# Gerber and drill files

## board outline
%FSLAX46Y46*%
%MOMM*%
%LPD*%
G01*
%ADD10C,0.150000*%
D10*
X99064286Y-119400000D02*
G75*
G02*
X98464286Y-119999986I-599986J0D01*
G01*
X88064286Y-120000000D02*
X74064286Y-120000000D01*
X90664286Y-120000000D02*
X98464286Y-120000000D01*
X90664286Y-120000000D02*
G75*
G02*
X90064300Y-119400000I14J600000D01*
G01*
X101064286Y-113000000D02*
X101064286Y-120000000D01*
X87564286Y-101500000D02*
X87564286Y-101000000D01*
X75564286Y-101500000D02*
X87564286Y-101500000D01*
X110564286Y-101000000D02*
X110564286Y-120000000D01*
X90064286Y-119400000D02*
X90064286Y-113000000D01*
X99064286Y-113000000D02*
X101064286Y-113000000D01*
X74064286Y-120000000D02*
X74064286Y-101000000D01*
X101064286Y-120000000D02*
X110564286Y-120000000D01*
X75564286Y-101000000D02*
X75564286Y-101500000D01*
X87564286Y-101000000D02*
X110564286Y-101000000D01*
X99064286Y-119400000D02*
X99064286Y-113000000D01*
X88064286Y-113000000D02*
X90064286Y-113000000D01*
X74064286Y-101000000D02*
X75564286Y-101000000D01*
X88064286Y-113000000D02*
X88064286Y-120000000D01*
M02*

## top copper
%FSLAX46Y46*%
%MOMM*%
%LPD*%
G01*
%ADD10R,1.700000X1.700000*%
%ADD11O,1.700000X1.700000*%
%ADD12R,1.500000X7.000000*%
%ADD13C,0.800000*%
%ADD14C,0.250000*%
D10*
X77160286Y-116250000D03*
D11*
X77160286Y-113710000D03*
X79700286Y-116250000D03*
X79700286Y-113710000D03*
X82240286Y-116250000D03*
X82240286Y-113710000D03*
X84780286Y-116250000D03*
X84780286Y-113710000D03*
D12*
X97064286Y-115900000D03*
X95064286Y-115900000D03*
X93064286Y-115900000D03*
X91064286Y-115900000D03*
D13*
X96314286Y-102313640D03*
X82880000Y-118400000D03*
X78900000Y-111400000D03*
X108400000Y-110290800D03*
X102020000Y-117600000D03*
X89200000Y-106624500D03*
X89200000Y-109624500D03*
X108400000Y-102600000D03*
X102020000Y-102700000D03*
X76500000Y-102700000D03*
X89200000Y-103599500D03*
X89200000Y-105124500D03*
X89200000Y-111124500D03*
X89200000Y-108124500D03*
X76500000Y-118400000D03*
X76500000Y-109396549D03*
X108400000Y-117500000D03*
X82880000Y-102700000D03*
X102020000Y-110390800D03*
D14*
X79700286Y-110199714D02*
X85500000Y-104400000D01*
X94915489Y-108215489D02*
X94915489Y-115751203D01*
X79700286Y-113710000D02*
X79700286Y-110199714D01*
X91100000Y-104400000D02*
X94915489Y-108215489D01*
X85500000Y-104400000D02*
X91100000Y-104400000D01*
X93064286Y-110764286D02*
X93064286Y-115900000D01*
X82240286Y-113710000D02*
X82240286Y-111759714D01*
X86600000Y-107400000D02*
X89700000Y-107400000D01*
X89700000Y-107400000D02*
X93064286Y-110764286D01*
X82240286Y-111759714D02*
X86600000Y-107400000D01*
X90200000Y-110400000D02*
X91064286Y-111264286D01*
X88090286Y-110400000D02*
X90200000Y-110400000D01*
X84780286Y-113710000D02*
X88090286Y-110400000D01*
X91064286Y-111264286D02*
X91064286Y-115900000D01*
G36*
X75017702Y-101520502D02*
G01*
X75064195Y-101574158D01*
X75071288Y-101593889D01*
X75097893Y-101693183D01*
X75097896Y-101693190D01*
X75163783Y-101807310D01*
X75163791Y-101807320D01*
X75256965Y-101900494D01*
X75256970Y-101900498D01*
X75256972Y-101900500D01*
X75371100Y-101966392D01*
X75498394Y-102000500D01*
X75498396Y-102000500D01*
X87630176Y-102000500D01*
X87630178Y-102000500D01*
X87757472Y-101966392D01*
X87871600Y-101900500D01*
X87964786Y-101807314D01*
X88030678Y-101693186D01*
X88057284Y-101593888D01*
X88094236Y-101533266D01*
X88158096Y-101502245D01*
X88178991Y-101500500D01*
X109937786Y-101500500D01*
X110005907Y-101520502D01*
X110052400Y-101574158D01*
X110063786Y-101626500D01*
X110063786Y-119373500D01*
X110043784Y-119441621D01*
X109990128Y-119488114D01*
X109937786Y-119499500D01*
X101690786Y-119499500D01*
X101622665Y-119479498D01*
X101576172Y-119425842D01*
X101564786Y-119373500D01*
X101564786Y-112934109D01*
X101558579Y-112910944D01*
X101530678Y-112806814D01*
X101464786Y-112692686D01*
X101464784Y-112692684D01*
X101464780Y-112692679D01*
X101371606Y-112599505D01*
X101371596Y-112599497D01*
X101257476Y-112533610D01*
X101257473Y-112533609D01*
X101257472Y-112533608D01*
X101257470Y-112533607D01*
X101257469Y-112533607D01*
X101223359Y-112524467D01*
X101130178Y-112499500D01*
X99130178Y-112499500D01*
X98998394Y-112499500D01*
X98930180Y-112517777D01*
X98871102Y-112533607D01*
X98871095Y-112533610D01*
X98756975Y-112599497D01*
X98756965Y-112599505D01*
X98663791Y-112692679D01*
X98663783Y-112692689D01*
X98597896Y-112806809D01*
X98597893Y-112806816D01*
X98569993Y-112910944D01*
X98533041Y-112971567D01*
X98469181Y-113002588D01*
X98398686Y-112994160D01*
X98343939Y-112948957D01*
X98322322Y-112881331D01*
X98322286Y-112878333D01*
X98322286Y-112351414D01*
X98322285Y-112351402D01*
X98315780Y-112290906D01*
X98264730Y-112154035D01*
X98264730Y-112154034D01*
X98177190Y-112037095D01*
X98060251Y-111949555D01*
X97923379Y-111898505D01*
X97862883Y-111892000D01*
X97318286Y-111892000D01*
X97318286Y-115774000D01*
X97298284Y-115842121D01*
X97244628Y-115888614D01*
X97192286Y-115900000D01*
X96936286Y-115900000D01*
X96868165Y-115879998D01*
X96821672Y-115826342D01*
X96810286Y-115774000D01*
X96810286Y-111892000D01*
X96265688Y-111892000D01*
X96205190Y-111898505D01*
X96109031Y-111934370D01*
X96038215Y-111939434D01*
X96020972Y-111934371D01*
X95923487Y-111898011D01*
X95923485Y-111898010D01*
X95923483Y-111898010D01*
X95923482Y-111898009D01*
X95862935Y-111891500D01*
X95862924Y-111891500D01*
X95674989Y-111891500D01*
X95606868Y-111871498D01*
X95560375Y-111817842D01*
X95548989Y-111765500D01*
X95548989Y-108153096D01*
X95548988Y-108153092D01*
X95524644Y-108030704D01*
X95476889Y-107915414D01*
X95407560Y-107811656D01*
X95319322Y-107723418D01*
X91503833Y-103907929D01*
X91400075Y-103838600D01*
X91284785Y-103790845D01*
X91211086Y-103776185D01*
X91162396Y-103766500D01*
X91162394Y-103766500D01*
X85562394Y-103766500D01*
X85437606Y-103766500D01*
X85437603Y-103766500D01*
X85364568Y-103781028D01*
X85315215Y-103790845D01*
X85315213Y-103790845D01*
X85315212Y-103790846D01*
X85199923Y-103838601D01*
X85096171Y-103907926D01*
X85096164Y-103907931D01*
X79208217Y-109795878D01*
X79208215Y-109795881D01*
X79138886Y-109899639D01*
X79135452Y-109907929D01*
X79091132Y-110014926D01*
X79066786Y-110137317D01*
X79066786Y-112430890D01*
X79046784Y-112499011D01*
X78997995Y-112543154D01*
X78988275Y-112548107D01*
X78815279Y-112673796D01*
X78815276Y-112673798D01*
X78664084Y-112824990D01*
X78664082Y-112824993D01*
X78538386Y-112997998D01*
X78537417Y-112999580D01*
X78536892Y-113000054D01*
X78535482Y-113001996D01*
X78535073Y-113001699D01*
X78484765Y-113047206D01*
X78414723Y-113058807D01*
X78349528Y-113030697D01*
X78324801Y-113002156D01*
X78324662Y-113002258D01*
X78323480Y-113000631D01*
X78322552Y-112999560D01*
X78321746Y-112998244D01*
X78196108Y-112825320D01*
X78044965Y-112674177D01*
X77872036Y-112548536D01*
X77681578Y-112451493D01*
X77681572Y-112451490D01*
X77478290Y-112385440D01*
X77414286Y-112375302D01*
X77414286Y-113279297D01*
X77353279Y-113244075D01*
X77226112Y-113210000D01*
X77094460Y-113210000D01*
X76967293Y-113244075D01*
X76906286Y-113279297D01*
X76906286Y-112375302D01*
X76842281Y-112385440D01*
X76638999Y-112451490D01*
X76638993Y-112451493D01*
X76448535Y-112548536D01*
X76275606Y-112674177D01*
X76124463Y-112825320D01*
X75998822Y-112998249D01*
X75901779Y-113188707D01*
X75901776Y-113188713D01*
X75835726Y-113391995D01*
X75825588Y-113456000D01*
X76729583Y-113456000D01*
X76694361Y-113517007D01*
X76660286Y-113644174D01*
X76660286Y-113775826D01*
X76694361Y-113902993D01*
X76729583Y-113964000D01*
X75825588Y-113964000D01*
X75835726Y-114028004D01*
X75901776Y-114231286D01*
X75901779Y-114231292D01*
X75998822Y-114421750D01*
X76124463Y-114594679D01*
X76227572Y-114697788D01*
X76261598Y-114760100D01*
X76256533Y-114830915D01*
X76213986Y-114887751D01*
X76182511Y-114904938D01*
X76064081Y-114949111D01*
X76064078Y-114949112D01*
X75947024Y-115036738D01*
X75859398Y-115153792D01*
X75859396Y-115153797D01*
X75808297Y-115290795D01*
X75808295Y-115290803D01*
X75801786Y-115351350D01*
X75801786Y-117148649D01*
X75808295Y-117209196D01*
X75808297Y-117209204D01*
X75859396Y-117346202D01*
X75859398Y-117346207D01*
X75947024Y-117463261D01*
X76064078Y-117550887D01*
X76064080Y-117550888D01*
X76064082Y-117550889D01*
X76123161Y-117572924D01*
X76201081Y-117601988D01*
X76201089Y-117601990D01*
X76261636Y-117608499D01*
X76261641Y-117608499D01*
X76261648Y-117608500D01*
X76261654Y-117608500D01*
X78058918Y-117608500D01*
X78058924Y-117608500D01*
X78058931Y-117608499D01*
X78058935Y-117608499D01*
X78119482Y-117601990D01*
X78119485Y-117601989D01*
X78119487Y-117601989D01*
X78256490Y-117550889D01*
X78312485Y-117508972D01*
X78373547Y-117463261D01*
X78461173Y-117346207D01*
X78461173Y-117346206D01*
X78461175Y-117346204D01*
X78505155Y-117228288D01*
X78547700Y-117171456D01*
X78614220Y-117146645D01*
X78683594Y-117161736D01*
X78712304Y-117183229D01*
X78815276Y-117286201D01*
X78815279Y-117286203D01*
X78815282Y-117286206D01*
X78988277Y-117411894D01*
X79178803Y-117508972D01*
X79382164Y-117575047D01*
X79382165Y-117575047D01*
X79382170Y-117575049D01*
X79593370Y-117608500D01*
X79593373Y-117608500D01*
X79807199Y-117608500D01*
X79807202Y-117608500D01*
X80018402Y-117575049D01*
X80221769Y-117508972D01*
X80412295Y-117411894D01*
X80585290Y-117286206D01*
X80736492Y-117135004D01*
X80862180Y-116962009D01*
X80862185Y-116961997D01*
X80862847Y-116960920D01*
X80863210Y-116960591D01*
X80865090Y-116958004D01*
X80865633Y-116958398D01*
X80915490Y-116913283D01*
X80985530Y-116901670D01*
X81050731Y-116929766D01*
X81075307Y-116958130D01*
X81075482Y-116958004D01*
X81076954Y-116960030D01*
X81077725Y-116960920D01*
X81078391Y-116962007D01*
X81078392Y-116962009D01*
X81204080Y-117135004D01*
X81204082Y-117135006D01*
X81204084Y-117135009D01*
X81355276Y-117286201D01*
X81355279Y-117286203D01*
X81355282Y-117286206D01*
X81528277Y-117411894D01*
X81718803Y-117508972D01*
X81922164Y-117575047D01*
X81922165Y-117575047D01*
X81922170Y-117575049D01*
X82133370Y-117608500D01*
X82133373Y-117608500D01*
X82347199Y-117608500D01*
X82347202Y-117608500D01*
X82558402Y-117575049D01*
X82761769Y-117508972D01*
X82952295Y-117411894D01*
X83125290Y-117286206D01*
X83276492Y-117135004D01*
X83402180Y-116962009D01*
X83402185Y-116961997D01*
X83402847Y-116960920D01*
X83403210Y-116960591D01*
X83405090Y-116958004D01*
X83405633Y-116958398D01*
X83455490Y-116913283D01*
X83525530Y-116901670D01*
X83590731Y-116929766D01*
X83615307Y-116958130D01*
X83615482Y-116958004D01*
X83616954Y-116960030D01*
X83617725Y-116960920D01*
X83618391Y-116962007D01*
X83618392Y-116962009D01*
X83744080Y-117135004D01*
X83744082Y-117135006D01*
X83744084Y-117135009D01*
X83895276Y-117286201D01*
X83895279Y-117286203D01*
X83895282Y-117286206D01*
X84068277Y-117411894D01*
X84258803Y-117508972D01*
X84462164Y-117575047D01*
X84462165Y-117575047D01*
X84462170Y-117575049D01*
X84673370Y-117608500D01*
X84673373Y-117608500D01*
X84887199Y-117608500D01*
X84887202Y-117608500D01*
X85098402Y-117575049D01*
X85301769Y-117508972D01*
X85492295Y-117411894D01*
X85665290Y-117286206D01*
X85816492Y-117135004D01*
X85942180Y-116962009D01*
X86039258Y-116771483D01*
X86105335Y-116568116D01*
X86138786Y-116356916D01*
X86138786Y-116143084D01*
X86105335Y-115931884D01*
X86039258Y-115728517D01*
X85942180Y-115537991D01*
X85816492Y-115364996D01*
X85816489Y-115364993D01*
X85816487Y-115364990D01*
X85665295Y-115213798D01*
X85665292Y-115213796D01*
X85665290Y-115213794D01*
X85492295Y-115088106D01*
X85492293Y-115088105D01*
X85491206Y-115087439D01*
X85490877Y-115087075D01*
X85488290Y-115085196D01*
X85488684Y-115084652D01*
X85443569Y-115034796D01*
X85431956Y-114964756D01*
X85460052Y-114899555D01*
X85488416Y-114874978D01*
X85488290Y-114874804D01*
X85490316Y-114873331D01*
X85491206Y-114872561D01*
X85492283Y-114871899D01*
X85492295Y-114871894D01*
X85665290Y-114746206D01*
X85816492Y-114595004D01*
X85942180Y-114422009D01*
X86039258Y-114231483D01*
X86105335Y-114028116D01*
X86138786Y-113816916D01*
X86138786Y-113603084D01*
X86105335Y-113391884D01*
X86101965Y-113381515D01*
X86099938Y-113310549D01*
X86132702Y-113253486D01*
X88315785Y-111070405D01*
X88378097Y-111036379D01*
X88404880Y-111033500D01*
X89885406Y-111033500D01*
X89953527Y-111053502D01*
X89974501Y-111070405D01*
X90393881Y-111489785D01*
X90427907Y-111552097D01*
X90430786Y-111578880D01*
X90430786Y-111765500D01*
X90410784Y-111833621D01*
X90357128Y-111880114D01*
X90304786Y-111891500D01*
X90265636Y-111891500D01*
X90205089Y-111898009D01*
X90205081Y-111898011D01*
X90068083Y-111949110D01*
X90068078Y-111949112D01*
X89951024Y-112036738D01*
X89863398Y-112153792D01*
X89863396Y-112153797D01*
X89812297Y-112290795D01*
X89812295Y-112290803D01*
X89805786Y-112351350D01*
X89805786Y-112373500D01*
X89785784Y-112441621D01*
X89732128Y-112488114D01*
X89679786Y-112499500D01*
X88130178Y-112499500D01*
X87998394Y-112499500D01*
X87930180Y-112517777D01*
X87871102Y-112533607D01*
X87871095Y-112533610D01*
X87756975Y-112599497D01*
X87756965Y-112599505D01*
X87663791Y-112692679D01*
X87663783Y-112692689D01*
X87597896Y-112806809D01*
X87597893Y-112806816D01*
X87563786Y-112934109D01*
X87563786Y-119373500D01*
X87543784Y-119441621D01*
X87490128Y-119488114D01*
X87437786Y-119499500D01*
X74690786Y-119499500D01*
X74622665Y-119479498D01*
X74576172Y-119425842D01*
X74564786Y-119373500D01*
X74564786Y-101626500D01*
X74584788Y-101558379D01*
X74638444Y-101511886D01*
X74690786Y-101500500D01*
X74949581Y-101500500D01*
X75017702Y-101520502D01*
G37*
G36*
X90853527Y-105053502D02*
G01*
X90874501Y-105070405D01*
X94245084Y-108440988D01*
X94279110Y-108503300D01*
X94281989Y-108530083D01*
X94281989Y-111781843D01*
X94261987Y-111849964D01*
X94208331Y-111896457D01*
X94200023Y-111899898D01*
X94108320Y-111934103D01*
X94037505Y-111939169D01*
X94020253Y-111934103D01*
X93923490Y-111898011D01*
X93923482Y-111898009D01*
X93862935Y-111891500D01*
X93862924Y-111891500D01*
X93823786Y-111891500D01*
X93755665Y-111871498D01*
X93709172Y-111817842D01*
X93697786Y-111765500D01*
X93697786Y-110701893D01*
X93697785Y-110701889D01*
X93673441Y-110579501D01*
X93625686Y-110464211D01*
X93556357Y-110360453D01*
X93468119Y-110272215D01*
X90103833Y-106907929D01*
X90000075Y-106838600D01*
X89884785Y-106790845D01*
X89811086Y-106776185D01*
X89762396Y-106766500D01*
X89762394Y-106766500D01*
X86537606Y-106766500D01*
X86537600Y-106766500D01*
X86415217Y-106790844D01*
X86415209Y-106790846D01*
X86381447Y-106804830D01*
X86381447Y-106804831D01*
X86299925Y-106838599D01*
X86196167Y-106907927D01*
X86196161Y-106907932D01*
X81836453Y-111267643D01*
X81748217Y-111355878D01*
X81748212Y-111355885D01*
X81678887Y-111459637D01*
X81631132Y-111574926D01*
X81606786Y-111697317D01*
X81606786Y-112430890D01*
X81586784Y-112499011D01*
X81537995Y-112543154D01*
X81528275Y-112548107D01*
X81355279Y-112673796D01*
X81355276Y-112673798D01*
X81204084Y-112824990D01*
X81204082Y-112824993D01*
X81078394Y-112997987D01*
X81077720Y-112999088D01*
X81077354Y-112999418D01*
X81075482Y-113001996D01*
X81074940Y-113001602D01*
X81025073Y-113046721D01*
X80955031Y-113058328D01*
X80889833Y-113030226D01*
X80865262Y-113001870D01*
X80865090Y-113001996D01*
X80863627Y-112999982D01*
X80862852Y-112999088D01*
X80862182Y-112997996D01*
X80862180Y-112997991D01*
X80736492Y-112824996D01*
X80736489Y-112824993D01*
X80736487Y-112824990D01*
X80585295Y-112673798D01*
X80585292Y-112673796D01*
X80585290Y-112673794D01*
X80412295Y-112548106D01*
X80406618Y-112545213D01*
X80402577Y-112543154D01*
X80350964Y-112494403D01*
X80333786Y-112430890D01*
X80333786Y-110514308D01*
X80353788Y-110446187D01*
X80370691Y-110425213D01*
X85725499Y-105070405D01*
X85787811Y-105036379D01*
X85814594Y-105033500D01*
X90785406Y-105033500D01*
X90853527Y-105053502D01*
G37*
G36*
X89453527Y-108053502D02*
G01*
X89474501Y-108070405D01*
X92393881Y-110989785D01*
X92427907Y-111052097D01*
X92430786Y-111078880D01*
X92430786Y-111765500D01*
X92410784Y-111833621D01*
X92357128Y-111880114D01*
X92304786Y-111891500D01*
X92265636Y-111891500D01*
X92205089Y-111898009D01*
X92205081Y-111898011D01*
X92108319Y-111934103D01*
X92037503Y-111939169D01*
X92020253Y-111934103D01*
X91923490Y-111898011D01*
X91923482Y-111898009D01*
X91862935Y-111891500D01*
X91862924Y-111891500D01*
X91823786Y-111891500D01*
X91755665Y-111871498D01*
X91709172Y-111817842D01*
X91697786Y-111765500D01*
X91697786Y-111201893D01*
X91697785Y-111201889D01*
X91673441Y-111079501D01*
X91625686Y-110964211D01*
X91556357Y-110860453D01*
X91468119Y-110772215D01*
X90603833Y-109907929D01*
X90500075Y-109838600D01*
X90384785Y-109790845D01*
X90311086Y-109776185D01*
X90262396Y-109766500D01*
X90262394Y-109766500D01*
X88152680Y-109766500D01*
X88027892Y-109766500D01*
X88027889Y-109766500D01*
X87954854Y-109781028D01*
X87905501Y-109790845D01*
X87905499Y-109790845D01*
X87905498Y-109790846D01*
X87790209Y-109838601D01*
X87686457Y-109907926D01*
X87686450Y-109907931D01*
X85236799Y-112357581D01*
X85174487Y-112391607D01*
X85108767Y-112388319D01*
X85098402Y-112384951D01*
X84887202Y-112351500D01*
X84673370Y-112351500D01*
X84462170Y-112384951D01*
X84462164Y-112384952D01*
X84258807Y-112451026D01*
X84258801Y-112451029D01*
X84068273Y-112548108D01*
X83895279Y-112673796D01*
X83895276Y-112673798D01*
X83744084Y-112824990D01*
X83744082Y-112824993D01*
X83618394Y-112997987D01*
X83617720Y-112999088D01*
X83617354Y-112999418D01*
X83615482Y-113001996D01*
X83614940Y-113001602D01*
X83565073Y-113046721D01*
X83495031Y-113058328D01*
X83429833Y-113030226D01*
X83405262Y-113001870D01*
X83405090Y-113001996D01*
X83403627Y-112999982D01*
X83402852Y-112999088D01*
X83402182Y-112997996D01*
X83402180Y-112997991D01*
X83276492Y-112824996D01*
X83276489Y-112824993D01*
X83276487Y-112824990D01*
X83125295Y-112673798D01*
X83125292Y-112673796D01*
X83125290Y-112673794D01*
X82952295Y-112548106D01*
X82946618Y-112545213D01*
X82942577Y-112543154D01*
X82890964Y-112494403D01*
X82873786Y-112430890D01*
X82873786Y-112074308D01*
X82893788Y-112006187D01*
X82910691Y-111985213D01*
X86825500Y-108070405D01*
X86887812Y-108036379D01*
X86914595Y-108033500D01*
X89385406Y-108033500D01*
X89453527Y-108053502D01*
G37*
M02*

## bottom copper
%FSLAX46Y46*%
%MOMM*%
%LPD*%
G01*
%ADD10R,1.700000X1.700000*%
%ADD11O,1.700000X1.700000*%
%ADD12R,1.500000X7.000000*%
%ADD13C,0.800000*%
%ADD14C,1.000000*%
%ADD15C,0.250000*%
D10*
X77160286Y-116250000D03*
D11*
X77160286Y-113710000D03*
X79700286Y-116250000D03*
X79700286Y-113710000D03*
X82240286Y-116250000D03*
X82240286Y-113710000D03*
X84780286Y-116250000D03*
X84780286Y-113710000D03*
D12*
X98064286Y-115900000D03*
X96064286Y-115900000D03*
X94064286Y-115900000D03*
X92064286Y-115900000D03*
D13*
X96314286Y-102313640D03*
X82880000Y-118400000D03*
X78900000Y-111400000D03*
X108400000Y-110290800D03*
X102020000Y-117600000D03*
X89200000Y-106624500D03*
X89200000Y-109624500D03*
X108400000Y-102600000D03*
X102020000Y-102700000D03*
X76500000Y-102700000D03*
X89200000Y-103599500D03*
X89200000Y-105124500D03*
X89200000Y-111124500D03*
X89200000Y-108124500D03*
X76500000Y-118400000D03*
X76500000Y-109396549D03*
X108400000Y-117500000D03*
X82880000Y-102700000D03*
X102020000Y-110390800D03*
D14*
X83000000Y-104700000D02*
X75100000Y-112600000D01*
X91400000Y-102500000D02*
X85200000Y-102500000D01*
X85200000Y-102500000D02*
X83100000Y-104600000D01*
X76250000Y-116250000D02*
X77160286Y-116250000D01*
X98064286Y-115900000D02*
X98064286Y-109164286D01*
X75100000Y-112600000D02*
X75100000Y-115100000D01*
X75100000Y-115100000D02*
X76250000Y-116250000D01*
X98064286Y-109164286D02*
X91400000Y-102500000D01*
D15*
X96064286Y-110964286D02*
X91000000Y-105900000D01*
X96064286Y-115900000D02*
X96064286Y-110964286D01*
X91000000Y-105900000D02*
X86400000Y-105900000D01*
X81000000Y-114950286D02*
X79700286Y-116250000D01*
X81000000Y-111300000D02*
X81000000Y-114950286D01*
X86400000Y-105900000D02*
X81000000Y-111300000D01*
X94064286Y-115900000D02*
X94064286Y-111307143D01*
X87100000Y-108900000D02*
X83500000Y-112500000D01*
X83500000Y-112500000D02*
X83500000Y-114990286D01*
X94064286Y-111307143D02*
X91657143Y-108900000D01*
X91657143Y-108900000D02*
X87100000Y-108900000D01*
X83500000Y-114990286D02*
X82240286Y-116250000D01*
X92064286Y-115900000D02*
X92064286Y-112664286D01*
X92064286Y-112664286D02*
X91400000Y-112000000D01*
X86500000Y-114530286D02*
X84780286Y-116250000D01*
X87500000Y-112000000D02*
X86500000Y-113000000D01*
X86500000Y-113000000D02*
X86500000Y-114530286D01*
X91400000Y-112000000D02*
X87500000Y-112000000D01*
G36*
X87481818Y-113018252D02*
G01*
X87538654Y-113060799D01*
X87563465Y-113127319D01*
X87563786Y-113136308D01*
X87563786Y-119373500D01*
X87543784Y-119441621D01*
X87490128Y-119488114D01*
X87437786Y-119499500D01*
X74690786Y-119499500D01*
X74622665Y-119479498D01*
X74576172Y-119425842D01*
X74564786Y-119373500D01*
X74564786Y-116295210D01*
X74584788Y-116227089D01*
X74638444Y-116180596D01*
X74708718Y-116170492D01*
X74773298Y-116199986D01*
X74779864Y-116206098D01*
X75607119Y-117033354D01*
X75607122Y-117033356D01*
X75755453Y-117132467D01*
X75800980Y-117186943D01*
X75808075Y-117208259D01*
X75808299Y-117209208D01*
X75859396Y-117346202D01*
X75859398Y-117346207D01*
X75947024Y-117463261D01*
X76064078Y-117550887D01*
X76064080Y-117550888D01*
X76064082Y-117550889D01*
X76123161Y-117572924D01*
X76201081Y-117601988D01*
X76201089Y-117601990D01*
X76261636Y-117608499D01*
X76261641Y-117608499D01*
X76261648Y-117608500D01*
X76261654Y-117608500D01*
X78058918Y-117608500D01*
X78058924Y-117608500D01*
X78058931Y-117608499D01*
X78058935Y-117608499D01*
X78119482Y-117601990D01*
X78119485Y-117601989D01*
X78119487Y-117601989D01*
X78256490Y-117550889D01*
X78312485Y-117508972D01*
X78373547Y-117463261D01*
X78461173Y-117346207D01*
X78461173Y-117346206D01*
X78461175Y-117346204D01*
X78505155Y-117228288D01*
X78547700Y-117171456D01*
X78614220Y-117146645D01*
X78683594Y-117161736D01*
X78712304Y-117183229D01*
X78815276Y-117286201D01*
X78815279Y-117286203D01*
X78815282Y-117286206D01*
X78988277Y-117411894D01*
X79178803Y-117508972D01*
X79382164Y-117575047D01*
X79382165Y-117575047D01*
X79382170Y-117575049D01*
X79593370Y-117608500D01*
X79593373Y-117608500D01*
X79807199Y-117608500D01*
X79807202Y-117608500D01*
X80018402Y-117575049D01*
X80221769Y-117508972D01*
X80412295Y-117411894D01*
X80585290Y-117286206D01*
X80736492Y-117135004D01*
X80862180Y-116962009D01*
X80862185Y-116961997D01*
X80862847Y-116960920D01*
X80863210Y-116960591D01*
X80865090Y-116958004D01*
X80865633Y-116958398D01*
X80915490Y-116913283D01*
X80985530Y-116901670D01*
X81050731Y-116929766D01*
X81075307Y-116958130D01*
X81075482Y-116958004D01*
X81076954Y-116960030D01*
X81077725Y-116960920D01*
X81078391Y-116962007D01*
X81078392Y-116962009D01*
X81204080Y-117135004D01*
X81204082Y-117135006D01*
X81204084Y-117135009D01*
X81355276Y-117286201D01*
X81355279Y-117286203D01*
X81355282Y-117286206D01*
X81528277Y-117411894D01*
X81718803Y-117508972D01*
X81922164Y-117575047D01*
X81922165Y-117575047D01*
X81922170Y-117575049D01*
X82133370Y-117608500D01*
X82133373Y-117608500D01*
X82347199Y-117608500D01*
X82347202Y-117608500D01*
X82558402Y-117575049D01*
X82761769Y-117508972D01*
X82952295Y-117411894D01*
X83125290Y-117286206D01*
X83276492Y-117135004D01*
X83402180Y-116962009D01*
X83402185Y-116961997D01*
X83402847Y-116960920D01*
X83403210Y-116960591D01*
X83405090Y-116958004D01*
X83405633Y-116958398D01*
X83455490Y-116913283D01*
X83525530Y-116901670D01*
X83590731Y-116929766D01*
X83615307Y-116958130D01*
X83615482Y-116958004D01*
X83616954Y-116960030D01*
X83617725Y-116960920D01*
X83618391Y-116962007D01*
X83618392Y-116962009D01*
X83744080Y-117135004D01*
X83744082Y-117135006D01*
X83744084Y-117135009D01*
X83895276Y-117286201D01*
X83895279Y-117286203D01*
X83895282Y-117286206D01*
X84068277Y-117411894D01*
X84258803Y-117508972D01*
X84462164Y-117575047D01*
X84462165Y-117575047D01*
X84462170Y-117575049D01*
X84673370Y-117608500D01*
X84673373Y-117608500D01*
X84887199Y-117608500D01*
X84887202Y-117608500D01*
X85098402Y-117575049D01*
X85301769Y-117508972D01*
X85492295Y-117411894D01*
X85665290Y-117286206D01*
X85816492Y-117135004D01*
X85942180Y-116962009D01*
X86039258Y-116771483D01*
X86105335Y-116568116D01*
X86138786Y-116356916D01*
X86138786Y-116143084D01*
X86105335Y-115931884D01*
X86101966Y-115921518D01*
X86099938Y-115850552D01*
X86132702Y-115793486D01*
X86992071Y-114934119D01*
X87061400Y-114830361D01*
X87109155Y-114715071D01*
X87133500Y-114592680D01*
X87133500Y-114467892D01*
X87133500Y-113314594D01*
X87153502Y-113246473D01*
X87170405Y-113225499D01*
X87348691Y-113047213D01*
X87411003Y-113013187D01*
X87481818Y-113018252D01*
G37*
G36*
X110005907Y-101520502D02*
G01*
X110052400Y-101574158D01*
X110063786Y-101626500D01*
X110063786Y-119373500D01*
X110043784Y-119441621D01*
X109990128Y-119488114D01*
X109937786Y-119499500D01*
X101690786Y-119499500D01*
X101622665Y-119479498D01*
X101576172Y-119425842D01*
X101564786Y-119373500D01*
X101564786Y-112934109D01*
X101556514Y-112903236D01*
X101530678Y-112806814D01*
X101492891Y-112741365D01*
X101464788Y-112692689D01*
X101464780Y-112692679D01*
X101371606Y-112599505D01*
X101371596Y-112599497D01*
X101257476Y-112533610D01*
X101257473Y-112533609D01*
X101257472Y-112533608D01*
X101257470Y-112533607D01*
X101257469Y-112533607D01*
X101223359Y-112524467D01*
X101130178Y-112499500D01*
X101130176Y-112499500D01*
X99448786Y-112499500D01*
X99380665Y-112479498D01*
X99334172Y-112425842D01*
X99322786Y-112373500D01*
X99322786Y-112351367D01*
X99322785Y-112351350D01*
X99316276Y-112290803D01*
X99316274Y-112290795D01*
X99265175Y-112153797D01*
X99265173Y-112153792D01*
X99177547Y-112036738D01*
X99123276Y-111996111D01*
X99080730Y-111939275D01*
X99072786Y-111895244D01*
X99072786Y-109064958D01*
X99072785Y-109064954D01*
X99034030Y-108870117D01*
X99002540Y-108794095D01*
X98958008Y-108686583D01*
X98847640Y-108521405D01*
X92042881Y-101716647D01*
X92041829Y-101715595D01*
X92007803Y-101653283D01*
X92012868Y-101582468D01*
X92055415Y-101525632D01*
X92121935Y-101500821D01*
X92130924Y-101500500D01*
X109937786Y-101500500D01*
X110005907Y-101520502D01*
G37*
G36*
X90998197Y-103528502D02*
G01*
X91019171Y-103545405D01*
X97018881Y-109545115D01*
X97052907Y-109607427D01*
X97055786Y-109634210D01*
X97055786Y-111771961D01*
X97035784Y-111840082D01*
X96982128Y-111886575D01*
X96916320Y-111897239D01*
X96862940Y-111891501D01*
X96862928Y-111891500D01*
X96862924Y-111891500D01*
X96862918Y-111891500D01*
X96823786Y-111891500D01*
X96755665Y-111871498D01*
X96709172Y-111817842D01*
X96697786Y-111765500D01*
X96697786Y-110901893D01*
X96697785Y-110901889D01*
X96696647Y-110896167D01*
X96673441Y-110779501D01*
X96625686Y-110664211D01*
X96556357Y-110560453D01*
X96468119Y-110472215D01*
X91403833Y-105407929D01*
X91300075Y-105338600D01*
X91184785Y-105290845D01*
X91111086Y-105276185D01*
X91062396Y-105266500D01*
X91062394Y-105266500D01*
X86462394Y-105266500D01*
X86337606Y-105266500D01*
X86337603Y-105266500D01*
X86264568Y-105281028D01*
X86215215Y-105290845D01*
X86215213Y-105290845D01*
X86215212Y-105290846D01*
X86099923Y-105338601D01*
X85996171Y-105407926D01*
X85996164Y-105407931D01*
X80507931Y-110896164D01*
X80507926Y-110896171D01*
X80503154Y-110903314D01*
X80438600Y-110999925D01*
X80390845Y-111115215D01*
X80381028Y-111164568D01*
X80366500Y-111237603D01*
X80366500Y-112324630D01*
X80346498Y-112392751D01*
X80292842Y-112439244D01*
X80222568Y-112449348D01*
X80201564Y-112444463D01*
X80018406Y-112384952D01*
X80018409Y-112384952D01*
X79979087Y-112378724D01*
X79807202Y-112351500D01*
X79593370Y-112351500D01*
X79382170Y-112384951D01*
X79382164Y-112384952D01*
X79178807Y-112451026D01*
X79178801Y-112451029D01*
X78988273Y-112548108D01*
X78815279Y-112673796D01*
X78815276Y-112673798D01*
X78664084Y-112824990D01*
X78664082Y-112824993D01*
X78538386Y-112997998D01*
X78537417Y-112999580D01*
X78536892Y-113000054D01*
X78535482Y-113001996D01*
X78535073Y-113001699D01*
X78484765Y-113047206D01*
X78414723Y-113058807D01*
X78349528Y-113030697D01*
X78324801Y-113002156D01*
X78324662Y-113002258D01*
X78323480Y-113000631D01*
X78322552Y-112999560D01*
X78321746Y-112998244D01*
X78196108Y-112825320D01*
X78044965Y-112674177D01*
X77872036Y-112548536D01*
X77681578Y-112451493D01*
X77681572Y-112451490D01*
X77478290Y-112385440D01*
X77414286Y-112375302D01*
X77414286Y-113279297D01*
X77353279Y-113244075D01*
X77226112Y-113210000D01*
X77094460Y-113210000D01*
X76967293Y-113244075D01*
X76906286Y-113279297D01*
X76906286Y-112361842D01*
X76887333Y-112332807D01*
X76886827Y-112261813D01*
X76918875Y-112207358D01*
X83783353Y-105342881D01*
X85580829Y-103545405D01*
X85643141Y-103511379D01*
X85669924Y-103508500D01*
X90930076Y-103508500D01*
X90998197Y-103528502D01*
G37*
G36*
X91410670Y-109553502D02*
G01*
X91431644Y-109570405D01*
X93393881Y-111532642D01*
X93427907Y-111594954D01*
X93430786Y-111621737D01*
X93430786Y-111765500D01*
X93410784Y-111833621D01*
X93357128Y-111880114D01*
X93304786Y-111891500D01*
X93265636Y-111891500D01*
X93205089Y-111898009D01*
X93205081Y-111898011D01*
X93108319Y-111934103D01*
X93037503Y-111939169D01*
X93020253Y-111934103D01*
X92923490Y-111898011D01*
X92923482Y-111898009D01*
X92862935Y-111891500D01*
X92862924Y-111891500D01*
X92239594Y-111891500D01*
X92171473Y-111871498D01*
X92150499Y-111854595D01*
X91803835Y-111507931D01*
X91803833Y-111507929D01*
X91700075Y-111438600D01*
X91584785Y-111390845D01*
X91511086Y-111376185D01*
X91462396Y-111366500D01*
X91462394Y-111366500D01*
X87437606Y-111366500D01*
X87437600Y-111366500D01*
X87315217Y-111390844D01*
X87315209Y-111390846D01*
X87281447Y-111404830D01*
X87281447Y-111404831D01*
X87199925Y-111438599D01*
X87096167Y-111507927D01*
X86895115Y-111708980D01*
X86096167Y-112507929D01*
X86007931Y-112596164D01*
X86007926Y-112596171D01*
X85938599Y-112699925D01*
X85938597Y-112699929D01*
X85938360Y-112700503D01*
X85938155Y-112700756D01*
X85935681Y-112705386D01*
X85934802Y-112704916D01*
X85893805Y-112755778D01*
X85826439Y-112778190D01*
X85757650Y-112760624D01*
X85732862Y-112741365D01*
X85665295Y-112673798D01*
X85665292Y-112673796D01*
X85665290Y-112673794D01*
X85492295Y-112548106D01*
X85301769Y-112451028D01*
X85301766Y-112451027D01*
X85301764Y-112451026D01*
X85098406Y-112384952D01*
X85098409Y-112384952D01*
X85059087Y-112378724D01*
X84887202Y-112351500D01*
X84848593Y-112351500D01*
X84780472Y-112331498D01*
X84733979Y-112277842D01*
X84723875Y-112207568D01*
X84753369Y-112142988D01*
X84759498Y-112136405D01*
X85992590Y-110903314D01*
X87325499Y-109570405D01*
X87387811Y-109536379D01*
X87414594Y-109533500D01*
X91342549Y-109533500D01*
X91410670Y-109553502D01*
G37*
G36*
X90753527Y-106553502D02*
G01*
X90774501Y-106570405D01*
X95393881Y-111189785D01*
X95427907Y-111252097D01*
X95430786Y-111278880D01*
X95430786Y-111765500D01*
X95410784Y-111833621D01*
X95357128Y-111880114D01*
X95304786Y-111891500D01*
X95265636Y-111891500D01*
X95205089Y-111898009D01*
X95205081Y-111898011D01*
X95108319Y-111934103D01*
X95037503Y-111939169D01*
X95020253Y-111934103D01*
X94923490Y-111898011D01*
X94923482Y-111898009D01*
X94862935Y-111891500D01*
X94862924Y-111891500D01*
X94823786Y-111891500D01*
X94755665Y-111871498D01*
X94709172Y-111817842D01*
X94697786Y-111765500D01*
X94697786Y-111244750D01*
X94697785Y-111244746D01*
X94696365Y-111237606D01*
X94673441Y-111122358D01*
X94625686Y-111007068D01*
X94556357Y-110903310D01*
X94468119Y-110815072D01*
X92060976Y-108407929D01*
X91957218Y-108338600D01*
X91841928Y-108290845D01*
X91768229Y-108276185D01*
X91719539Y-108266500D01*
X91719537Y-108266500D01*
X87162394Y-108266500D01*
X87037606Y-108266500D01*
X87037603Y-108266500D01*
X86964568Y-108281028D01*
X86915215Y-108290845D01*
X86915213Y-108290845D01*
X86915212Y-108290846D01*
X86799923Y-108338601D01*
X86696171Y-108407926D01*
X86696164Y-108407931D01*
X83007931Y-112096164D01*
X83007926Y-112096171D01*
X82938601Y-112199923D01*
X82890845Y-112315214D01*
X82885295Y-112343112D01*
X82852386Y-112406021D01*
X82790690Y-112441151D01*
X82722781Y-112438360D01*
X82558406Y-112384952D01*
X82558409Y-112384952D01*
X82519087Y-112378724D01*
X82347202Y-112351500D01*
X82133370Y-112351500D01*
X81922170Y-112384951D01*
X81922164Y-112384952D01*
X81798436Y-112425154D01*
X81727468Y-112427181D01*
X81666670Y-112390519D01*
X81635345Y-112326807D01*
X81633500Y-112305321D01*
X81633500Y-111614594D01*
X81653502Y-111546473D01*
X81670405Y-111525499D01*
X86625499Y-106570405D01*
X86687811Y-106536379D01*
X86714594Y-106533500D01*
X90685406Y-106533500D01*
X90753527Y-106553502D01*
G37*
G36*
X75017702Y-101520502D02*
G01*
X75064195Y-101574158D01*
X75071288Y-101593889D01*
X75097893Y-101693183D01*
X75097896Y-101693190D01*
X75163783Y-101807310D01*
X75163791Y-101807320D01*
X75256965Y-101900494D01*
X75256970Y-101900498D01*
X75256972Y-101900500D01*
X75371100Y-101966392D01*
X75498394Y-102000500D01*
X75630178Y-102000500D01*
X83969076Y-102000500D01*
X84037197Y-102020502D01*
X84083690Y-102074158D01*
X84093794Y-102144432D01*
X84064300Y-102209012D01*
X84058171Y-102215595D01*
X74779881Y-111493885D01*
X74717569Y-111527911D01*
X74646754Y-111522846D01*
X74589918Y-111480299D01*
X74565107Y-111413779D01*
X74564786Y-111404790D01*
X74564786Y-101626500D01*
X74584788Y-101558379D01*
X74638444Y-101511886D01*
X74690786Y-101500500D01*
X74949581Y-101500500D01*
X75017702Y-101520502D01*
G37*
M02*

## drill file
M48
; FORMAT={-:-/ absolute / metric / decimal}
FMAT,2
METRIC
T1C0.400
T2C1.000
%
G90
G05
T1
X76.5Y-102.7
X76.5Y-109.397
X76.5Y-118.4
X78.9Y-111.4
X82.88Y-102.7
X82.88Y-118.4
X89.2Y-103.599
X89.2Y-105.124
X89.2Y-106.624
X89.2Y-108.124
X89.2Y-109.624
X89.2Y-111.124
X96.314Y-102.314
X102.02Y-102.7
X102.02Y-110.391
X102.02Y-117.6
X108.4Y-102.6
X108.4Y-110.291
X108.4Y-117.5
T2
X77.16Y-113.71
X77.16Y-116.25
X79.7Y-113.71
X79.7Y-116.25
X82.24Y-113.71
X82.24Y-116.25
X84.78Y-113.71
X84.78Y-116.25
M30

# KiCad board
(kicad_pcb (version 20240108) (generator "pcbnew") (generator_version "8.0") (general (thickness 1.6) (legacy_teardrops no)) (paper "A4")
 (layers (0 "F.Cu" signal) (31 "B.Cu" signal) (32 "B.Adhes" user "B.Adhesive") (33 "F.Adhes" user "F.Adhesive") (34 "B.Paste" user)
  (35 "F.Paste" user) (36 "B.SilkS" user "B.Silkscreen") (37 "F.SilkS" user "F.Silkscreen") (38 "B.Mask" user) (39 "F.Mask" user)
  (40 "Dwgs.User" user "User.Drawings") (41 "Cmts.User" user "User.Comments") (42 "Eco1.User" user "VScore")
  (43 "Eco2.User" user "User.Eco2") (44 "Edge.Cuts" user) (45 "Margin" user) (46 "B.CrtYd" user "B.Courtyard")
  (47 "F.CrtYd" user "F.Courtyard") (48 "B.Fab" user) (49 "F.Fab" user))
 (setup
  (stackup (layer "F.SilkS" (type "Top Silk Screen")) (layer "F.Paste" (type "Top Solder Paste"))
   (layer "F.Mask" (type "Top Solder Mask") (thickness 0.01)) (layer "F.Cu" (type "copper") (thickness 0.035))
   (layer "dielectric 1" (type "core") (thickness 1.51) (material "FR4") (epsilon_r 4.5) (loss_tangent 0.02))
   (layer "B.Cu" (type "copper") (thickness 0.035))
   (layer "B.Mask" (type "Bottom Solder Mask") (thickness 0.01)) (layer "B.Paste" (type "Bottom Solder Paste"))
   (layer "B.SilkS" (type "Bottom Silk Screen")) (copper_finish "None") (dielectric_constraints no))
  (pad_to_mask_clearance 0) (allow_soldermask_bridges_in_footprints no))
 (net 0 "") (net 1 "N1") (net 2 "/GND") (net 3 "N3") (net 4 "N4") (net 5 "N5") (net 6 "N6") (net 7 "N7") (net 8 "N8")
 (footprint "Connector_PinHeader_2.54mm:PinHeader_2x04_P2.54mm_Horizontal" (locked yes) (layer "F.Cu") (at 77.160286 116.25 90)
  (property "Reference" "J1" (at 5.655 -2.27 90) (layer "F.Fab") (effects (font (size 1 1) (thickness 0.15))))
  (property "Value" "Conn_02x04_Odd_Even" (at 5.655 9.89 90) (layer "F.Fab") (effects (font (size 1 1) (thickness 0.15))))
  (pad "1" thru_hole rect (at 0 0 90) (size 1.7 1.7) (drill 1) (layers "*.Cu" "*.Mask") (remove_unused_layers no) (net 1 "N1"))
  (pad "2" thru_hole oval (at 2.54 0 90) (size 1.7 1.7) (drill 1) (layers "*.Cu" "*.Mask") (remove_unused_layers no) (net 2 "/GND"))
  (pad "3" thru_hole oval (at 0 2.54 90) (size 1.7 1.7) (drill 1) (layers "*.Cu" "*.Mask") (remove_unused_layers no) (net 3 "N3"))
  (pad "4" thru_hole oval (at 2.54 2.54 90) (size 1.7 1.7) (drill 1) (layers "*.Cu" "*.Mask") (remove_unused_layers no) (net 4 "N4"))
  (pad "5" thru_hole oval (at 0 5.08 90) (size 1.7 1.7) (drill 1) (layers "*.Cu" "*.Mask") (remove_unused_layers no) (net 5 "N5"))
  (pad "6" thru_hole oval (at 2.54 5.08 90) (size 1.7 1.7) (drill 1) (layers "*.Cu" "*.Mask") (remove_unused_layers no) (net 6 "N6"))
  (pad "7" thru_hole oval (at 0 7.62 90) (size 1.7 1.7) (drill 1) (layers "*.Cu" "*.Mask") (remove_unused_layers no) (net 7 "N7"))
  (pad "8" thru_hole oval (at 2.54 7.62 90) (size 1.7 1.7) (drill 1) (layers "*.Cu" "*.Mask") (remove_unused_layers no) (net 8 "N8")))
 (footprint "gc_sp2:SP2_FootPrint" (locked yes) (layer "B.Cu") (at 98.064286 115.9 180)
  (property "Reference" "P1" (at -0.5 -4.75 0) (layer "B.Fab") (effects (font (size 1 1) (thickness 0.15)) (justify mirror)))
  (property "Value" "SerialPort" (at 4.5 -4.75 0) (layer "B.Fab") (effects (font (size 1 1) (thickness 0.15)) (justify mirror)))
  (pad "1" smd rect (at 0 0 180) (size 1.5 7) (layers "B.Cu" "B.Paste" "B.Mask") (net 1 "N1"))
  (pad "2" smd rect (at 1 0 180) (size 1.5 7) (layers "F.Cu" "F.Paste" "F.Mask") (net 2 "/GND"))
  (pad "3" smd rect (at 2 0 180) (size 1.5 7) (layers "B.Cu" "B.Paste" "B.Mask") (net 3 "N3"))
  (pad "4" smd rect (at 3 0 180) (size 1.5 7) (layers "F.Cu" "F.Paste" "F.Mask") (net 4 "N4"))
  (pad "5" smd rect (at 4 0 180) (size 1.5 7) (layers "B.Cu" "B.Paste" "B.Mask") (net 5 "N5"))
  (pad "6" smd rect (at 5 0 180) (size 1.5 7) (layers "F.Cu" "F.Paste" "F.Mask") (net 6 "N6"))
  (pad "7" smd rect (at 6 0 180) (size 1.5 7) (layers "B.Cu" "B.Paste" "B.Mask") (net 7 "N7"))
  (pad "8" smd rect (at 7 0 180) (size 1.5 7) (layers "F.Cu" "F.Paste" "F.Mask") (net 8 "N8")))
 (gr_arc (start 99.064286 119.4) (mid 98.88855 119.824264) (end 98.464286 120) (stroke (width 0.15) (type solid)) (layer "Edge.Cuts"))
 (gr_line (start 88.064286 120) (end 74.064286 120) (stroke (width 0.15) (type solid)) (layer "Edge.Cuts"))
 (gr_line (start 90.664286 120) (end 98.464286 120) (stroke (width 0.15) (type solid)) (layer "Edge.Cuts"))
 (gr_arc (start 90.664286 120) (mid 90.240022 119.824264) (end 90.064286 119.4) (stroke (width 0.15) (type solid)) (layer "Edge.Cuts"))
 (gr_line (start 101.064286 113) (end 101.064286 120) (stroke (width 0.15) (type solid)) (layer "Edge.Cuts"))
 (gr_line (start 87.564286 101.5) (end 87.564286 101) (stroke (width 0.15) (type default)) (layer "Edge.Cuts"))
 (gr_line (start 75.564286 101.5) (end 87.564286 101.5) (stroke (width 0.15) (type default)) (layer "Edge.Cuts"))
 (gr_line (start 110.564286 101) (end 110.564286 120) (stroke (width 0.15) (type solid)) (layer "Edge.Cuts"))
 (gr_line (start 90.064286 119.4) (end 90.064286 113) (stroke (width 0.15) (type solid)) (layer "Edge.Cuts"))
 (gr_line (start 99.064286 113) (end 101.064286 113) (stroke (width 0.15) (type solid)) (layer "Edge.Cuts"))
 (gr_line (start 74.064286 120) (end 74.064286 101) (stroke (width 0.15) (type solid)) (layer "Edge.Cuts"))
 (gr_line (start 101.064286 120) (end 110.564286 120) (stroke (width 0.15) (type solid)) (layer "Edge.Cuts"))
 (gr_line (start 75.564286 101) (end 75.564286 101.5) (stroke (width 0.15) (type default)) (layer "Edge.Cuts"))
 (gr_line (start 87.564286 101) (end 110.564286 101) (stroke (width 0.15) (type solid)) (layer "Edge.Cuts"))
 (gr_line (start 99.064286 119.4) (end 99.064286 113) (stroke (width 0.15) (type solid)) (layer "Edge.Cuts"))
 (gr_line (start 88.064286 113) (end 90.064286 113) (stroke (width 0.15) (type solid)) (layer "Edge.Cuts"))
 (gr_line (start 74.064286 101) (end 75.564286 101) (stroke (width 0.15) (type default)) (layer "Edge.Cuts"))
 (gr_line (start 88.064286 113) (end 88.064286 120) (stroke (width 0.15) (type solid)) (layer "Edge.Cuts"))
 (segment (start 83 104.7) (end 75.1 112.6) (width 1) (layer "B.Cu") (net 1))
 (segment (start 91.4 102.5) (end 85.2 102.5) (width 1) (layer "B.Cu") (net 1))
 (segment (start 85.2 102.5) (end 83.1 104.6) (width 1) (layer "B.Cu") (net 1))
 (segment (start 76.25 116.25) (end 77.160286 116.25) (width 1) (layer "B.Cu") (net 1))
 (segment (start 98.064286 115.9) (end 98.064286 109.164286) (width 1) (layer "B.Cu") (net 1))
 (segment (start 75.1 112.6) (end 75.1 115.1) (width 1) (layer "B.Cu") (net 1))
 (segment (start 75.1 115.1) (end 76.25 116.25) (width 1) (layer "B.Cu") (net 1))
 (segment (start 98.064286 109.164286) (end 91.4 102.5) (width 1) (layer "B.Cu") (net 1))
 (segment (start 96.064286 110.964286) (end 91 105.9) (width 0.25) (layer "B.Cu") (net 3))
 (segment (start 96.064286 115.9) (end 96.064286 110.964286) (width 0.25) (layer "B.Cu") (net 3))
 (segment (start 91 105.9) (end 86.4 105.9) (width 0.25) (layer "B.Cu") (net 3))
 (segment (start 81 114.950286) (end 79.700286 116.25) (width 0.25) (layer "B.Cu") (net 3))
 (segment (start 81 111.3) (end 81 114.950286) (width 0.25) (layer "B.Cu") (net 3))
 (segment (start 86.4 105.9) (end 81 111.3) (width 0.25) (layer "B.Cu") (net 3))
 (segment (start 79.700286 110.199714) (end 85.5 104.4) (width 0.25) (layer "F.Cu") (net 4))
 (segment (start 94.915489 108.215489) (end 94.915489 115.751203) (width 0.25) (layer "F.Cu") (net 4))
 (segment (start 79.700286 113.71) (end 79.700286 110.199714) (width 0.25) (layer "F.Cu") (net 4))
 (segment (start 91.1 104.4) (end 94.915489 108.215489) (width 0.25) (layer "F.Cu") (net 4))
 (segment (start 85.5 104.4) (end 91.1 104.4) (width 0.25) (layer "F.Cu") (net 4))
 (segment (start 94.064286 115.9) (end 94.064286 111.307143) (width 0.25) (layer "B.Cu") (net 5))
 (segment (start 87.1 108.9) (end 83.5 112.5) (width 0.25) (layer "B.Cu") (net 5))
 (segment (start 83.5 112.5) (end 83.5 114.990286) (width 0.25) (layer "B.Cu") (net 5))
 (segment (start 94.064286 111.307143) (end 91.657143 108.9) (width 0.25) (layer "B.Cu") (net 5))
 (segment (start 91.657143 108.9) (end 87.1 108.9) (width 0.25) (layer "B.Cu") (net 5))
 (segment (start 83.5 114.990286) (end 82.240286 116.25) (width 0.25) (layer "B.Cu") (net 5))
 (segment (start 93.064286 110.764286) (end 93.064286 115.9) (width 0.25) (layer "F.Cu") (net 6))
 (segment (start 82.240286 113.71) (end 82.240286 111.759714) (width 0.25) (layer "F.Cu") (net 6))
 (segment (start 86.6 107.4) (end 89.7 107.4) (width 0.25) (layer "F.Cu") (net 6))
 (segment (start 89.7 107.4) (end 93.064286 110.764286) (width 0.25) (layer "F.Cu") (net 6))
 (segment (start 82.240286 111.759714) (end 86.6 107.4) (width 0.25) (layer "F.Cu") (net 6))
 (segment (start 92.064286 115.9) (end 92.064286 112.664286) (width 0.25) (layer "B.Cu") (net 7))
 (segment (start 92.064286 112.664286) (end 91.4 112) (width 0.25) (layer "B.Cu") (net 7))
 (segment (start 86.5 114.530286) (end 84.780286 116.25) (width 0.25) (layer "B.Cu") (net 7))
 (segment (start 87.5 112) (end 86.5 113) (width 0.25) (layer "B.Cu") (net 7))
 (segment (start 86.5 113) (end 86.5 114.530286) (width 0.25) (layer "B.Cu") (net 7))
 (segment (start 91.4 112) (end 87.5 112) (width 0.25) (layer "B.Cu") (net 7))
 (segment (start 90.2 110.4) (end 91.064286 111.264286) (width 0.25) (layer "F.Cu") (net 8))
 (segment (start 88.090286 110.4) (end 90.2 110.4) (width 0.25) (layer "F.Cu") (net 8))
 (segment (start 84.780286 113.71) (end 88.090286 110.4) (width 0.25) (layer "F.Cu") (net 8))
 (segment (start 91.064286 111.264286) (end 91.064286 115.9) (width 0.25) (layer "F.Cu") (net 8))
 (via (at 96.314286 102.31364) (size 0.8) (drill 0.4) (layers "F.Cu" "B.Cu") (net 2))
 (via (at 82.88 118.4) (size 0.8) (drill 0.4) (layers "F.Cu" "B.Cu") (free yes) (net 2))
 (via (at 78.9 111.4) (size 0.8) (drill 0.4) (layers "F.Cu" "B.Cu") (free yes) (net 2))
 (via (at 108.4 110.2908) (size 0.8) (drill 0.4) (layers "F.Cu" "B.Cu") (free yes) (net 2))
 (via (at 102.02 117.6) (size 0.8) (drill 0.4) (layers "F.Cu" "B.Cu") (free yes) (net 2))
 (via (at 89.2 106.6245) (size 0.8) (drill 0.4) (layers "F.Cu" "B.Cu") (free yes) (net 2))
 (via (at 89.2 109.6245) (size 0.8) (drill 0.4) (layers "F.Cu" "B.Cu") (free yes) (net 2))
 (via (at 108.4 102.6) (size 0.8) (drill 0.4) (layers "F.Cu" "B.Cu") (free yes) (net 2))
 (via (at 102.02 102.7) (size 0.8) (drill 0.4) (layers "F.Cu" "B.Cu") (free yes) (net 2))
 (via (at 76.5 102.7) (size 0.8) (drill 0.4) (layers "F.Cu" "B.Cu") (free yes) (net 2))
 (via (at 89.2 103.5995) (size 0.8) (drill 0.4) (layers "F.Cu" "B.Cu") (free yes) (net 2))
 (via (at 89.2 105.1245) (size 0.8) (drill 0.4) (layers "F.Cu" "B.Cu") (free yes) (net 2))
 (via (at 89.2 111.1245) (size 0.8) (drill 0.4) (layers "F.Cu" "B.Cu") (free yes) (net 2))
 (via (at 89.2 108.1245) (size 0.8) (drill 0.4) (layers "F.Cu" "B.Cu") (free yes) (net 2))
 (via (at 76.5 118.4) (size 0.8) (drill 0.4) (layers "F.Cu" "B.Cu") (free yes) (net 2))
 (via (at 76.5 109.396549) (size 0.8) (drill 0.4) (layers "F.Cu" "B.Cu") (free yes) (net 2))
 (via (at 108.4 117.5) (size 0.8) (drill 0.4) (layers "F.Cu" "B.Cu") (free yes) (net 2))
 (via (at 82.88 102.7) (size 0.8) (drill 0.4) (layers "F.Cu" "B.Cu") (free yes) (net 2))
 (via (at 102.02 110.3908) (size 0.8) (drill 0.4) (layers "F.Cu" "B.Cu") (free yes) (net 2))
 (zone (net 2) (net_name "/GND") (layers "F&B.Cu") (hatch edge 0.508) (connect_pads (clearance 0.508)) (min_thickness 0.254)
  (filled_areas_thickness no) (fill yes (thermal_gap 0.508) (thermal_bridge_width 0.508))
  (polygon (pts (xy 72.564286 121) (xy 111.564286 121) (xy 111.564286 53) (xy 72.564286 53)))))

